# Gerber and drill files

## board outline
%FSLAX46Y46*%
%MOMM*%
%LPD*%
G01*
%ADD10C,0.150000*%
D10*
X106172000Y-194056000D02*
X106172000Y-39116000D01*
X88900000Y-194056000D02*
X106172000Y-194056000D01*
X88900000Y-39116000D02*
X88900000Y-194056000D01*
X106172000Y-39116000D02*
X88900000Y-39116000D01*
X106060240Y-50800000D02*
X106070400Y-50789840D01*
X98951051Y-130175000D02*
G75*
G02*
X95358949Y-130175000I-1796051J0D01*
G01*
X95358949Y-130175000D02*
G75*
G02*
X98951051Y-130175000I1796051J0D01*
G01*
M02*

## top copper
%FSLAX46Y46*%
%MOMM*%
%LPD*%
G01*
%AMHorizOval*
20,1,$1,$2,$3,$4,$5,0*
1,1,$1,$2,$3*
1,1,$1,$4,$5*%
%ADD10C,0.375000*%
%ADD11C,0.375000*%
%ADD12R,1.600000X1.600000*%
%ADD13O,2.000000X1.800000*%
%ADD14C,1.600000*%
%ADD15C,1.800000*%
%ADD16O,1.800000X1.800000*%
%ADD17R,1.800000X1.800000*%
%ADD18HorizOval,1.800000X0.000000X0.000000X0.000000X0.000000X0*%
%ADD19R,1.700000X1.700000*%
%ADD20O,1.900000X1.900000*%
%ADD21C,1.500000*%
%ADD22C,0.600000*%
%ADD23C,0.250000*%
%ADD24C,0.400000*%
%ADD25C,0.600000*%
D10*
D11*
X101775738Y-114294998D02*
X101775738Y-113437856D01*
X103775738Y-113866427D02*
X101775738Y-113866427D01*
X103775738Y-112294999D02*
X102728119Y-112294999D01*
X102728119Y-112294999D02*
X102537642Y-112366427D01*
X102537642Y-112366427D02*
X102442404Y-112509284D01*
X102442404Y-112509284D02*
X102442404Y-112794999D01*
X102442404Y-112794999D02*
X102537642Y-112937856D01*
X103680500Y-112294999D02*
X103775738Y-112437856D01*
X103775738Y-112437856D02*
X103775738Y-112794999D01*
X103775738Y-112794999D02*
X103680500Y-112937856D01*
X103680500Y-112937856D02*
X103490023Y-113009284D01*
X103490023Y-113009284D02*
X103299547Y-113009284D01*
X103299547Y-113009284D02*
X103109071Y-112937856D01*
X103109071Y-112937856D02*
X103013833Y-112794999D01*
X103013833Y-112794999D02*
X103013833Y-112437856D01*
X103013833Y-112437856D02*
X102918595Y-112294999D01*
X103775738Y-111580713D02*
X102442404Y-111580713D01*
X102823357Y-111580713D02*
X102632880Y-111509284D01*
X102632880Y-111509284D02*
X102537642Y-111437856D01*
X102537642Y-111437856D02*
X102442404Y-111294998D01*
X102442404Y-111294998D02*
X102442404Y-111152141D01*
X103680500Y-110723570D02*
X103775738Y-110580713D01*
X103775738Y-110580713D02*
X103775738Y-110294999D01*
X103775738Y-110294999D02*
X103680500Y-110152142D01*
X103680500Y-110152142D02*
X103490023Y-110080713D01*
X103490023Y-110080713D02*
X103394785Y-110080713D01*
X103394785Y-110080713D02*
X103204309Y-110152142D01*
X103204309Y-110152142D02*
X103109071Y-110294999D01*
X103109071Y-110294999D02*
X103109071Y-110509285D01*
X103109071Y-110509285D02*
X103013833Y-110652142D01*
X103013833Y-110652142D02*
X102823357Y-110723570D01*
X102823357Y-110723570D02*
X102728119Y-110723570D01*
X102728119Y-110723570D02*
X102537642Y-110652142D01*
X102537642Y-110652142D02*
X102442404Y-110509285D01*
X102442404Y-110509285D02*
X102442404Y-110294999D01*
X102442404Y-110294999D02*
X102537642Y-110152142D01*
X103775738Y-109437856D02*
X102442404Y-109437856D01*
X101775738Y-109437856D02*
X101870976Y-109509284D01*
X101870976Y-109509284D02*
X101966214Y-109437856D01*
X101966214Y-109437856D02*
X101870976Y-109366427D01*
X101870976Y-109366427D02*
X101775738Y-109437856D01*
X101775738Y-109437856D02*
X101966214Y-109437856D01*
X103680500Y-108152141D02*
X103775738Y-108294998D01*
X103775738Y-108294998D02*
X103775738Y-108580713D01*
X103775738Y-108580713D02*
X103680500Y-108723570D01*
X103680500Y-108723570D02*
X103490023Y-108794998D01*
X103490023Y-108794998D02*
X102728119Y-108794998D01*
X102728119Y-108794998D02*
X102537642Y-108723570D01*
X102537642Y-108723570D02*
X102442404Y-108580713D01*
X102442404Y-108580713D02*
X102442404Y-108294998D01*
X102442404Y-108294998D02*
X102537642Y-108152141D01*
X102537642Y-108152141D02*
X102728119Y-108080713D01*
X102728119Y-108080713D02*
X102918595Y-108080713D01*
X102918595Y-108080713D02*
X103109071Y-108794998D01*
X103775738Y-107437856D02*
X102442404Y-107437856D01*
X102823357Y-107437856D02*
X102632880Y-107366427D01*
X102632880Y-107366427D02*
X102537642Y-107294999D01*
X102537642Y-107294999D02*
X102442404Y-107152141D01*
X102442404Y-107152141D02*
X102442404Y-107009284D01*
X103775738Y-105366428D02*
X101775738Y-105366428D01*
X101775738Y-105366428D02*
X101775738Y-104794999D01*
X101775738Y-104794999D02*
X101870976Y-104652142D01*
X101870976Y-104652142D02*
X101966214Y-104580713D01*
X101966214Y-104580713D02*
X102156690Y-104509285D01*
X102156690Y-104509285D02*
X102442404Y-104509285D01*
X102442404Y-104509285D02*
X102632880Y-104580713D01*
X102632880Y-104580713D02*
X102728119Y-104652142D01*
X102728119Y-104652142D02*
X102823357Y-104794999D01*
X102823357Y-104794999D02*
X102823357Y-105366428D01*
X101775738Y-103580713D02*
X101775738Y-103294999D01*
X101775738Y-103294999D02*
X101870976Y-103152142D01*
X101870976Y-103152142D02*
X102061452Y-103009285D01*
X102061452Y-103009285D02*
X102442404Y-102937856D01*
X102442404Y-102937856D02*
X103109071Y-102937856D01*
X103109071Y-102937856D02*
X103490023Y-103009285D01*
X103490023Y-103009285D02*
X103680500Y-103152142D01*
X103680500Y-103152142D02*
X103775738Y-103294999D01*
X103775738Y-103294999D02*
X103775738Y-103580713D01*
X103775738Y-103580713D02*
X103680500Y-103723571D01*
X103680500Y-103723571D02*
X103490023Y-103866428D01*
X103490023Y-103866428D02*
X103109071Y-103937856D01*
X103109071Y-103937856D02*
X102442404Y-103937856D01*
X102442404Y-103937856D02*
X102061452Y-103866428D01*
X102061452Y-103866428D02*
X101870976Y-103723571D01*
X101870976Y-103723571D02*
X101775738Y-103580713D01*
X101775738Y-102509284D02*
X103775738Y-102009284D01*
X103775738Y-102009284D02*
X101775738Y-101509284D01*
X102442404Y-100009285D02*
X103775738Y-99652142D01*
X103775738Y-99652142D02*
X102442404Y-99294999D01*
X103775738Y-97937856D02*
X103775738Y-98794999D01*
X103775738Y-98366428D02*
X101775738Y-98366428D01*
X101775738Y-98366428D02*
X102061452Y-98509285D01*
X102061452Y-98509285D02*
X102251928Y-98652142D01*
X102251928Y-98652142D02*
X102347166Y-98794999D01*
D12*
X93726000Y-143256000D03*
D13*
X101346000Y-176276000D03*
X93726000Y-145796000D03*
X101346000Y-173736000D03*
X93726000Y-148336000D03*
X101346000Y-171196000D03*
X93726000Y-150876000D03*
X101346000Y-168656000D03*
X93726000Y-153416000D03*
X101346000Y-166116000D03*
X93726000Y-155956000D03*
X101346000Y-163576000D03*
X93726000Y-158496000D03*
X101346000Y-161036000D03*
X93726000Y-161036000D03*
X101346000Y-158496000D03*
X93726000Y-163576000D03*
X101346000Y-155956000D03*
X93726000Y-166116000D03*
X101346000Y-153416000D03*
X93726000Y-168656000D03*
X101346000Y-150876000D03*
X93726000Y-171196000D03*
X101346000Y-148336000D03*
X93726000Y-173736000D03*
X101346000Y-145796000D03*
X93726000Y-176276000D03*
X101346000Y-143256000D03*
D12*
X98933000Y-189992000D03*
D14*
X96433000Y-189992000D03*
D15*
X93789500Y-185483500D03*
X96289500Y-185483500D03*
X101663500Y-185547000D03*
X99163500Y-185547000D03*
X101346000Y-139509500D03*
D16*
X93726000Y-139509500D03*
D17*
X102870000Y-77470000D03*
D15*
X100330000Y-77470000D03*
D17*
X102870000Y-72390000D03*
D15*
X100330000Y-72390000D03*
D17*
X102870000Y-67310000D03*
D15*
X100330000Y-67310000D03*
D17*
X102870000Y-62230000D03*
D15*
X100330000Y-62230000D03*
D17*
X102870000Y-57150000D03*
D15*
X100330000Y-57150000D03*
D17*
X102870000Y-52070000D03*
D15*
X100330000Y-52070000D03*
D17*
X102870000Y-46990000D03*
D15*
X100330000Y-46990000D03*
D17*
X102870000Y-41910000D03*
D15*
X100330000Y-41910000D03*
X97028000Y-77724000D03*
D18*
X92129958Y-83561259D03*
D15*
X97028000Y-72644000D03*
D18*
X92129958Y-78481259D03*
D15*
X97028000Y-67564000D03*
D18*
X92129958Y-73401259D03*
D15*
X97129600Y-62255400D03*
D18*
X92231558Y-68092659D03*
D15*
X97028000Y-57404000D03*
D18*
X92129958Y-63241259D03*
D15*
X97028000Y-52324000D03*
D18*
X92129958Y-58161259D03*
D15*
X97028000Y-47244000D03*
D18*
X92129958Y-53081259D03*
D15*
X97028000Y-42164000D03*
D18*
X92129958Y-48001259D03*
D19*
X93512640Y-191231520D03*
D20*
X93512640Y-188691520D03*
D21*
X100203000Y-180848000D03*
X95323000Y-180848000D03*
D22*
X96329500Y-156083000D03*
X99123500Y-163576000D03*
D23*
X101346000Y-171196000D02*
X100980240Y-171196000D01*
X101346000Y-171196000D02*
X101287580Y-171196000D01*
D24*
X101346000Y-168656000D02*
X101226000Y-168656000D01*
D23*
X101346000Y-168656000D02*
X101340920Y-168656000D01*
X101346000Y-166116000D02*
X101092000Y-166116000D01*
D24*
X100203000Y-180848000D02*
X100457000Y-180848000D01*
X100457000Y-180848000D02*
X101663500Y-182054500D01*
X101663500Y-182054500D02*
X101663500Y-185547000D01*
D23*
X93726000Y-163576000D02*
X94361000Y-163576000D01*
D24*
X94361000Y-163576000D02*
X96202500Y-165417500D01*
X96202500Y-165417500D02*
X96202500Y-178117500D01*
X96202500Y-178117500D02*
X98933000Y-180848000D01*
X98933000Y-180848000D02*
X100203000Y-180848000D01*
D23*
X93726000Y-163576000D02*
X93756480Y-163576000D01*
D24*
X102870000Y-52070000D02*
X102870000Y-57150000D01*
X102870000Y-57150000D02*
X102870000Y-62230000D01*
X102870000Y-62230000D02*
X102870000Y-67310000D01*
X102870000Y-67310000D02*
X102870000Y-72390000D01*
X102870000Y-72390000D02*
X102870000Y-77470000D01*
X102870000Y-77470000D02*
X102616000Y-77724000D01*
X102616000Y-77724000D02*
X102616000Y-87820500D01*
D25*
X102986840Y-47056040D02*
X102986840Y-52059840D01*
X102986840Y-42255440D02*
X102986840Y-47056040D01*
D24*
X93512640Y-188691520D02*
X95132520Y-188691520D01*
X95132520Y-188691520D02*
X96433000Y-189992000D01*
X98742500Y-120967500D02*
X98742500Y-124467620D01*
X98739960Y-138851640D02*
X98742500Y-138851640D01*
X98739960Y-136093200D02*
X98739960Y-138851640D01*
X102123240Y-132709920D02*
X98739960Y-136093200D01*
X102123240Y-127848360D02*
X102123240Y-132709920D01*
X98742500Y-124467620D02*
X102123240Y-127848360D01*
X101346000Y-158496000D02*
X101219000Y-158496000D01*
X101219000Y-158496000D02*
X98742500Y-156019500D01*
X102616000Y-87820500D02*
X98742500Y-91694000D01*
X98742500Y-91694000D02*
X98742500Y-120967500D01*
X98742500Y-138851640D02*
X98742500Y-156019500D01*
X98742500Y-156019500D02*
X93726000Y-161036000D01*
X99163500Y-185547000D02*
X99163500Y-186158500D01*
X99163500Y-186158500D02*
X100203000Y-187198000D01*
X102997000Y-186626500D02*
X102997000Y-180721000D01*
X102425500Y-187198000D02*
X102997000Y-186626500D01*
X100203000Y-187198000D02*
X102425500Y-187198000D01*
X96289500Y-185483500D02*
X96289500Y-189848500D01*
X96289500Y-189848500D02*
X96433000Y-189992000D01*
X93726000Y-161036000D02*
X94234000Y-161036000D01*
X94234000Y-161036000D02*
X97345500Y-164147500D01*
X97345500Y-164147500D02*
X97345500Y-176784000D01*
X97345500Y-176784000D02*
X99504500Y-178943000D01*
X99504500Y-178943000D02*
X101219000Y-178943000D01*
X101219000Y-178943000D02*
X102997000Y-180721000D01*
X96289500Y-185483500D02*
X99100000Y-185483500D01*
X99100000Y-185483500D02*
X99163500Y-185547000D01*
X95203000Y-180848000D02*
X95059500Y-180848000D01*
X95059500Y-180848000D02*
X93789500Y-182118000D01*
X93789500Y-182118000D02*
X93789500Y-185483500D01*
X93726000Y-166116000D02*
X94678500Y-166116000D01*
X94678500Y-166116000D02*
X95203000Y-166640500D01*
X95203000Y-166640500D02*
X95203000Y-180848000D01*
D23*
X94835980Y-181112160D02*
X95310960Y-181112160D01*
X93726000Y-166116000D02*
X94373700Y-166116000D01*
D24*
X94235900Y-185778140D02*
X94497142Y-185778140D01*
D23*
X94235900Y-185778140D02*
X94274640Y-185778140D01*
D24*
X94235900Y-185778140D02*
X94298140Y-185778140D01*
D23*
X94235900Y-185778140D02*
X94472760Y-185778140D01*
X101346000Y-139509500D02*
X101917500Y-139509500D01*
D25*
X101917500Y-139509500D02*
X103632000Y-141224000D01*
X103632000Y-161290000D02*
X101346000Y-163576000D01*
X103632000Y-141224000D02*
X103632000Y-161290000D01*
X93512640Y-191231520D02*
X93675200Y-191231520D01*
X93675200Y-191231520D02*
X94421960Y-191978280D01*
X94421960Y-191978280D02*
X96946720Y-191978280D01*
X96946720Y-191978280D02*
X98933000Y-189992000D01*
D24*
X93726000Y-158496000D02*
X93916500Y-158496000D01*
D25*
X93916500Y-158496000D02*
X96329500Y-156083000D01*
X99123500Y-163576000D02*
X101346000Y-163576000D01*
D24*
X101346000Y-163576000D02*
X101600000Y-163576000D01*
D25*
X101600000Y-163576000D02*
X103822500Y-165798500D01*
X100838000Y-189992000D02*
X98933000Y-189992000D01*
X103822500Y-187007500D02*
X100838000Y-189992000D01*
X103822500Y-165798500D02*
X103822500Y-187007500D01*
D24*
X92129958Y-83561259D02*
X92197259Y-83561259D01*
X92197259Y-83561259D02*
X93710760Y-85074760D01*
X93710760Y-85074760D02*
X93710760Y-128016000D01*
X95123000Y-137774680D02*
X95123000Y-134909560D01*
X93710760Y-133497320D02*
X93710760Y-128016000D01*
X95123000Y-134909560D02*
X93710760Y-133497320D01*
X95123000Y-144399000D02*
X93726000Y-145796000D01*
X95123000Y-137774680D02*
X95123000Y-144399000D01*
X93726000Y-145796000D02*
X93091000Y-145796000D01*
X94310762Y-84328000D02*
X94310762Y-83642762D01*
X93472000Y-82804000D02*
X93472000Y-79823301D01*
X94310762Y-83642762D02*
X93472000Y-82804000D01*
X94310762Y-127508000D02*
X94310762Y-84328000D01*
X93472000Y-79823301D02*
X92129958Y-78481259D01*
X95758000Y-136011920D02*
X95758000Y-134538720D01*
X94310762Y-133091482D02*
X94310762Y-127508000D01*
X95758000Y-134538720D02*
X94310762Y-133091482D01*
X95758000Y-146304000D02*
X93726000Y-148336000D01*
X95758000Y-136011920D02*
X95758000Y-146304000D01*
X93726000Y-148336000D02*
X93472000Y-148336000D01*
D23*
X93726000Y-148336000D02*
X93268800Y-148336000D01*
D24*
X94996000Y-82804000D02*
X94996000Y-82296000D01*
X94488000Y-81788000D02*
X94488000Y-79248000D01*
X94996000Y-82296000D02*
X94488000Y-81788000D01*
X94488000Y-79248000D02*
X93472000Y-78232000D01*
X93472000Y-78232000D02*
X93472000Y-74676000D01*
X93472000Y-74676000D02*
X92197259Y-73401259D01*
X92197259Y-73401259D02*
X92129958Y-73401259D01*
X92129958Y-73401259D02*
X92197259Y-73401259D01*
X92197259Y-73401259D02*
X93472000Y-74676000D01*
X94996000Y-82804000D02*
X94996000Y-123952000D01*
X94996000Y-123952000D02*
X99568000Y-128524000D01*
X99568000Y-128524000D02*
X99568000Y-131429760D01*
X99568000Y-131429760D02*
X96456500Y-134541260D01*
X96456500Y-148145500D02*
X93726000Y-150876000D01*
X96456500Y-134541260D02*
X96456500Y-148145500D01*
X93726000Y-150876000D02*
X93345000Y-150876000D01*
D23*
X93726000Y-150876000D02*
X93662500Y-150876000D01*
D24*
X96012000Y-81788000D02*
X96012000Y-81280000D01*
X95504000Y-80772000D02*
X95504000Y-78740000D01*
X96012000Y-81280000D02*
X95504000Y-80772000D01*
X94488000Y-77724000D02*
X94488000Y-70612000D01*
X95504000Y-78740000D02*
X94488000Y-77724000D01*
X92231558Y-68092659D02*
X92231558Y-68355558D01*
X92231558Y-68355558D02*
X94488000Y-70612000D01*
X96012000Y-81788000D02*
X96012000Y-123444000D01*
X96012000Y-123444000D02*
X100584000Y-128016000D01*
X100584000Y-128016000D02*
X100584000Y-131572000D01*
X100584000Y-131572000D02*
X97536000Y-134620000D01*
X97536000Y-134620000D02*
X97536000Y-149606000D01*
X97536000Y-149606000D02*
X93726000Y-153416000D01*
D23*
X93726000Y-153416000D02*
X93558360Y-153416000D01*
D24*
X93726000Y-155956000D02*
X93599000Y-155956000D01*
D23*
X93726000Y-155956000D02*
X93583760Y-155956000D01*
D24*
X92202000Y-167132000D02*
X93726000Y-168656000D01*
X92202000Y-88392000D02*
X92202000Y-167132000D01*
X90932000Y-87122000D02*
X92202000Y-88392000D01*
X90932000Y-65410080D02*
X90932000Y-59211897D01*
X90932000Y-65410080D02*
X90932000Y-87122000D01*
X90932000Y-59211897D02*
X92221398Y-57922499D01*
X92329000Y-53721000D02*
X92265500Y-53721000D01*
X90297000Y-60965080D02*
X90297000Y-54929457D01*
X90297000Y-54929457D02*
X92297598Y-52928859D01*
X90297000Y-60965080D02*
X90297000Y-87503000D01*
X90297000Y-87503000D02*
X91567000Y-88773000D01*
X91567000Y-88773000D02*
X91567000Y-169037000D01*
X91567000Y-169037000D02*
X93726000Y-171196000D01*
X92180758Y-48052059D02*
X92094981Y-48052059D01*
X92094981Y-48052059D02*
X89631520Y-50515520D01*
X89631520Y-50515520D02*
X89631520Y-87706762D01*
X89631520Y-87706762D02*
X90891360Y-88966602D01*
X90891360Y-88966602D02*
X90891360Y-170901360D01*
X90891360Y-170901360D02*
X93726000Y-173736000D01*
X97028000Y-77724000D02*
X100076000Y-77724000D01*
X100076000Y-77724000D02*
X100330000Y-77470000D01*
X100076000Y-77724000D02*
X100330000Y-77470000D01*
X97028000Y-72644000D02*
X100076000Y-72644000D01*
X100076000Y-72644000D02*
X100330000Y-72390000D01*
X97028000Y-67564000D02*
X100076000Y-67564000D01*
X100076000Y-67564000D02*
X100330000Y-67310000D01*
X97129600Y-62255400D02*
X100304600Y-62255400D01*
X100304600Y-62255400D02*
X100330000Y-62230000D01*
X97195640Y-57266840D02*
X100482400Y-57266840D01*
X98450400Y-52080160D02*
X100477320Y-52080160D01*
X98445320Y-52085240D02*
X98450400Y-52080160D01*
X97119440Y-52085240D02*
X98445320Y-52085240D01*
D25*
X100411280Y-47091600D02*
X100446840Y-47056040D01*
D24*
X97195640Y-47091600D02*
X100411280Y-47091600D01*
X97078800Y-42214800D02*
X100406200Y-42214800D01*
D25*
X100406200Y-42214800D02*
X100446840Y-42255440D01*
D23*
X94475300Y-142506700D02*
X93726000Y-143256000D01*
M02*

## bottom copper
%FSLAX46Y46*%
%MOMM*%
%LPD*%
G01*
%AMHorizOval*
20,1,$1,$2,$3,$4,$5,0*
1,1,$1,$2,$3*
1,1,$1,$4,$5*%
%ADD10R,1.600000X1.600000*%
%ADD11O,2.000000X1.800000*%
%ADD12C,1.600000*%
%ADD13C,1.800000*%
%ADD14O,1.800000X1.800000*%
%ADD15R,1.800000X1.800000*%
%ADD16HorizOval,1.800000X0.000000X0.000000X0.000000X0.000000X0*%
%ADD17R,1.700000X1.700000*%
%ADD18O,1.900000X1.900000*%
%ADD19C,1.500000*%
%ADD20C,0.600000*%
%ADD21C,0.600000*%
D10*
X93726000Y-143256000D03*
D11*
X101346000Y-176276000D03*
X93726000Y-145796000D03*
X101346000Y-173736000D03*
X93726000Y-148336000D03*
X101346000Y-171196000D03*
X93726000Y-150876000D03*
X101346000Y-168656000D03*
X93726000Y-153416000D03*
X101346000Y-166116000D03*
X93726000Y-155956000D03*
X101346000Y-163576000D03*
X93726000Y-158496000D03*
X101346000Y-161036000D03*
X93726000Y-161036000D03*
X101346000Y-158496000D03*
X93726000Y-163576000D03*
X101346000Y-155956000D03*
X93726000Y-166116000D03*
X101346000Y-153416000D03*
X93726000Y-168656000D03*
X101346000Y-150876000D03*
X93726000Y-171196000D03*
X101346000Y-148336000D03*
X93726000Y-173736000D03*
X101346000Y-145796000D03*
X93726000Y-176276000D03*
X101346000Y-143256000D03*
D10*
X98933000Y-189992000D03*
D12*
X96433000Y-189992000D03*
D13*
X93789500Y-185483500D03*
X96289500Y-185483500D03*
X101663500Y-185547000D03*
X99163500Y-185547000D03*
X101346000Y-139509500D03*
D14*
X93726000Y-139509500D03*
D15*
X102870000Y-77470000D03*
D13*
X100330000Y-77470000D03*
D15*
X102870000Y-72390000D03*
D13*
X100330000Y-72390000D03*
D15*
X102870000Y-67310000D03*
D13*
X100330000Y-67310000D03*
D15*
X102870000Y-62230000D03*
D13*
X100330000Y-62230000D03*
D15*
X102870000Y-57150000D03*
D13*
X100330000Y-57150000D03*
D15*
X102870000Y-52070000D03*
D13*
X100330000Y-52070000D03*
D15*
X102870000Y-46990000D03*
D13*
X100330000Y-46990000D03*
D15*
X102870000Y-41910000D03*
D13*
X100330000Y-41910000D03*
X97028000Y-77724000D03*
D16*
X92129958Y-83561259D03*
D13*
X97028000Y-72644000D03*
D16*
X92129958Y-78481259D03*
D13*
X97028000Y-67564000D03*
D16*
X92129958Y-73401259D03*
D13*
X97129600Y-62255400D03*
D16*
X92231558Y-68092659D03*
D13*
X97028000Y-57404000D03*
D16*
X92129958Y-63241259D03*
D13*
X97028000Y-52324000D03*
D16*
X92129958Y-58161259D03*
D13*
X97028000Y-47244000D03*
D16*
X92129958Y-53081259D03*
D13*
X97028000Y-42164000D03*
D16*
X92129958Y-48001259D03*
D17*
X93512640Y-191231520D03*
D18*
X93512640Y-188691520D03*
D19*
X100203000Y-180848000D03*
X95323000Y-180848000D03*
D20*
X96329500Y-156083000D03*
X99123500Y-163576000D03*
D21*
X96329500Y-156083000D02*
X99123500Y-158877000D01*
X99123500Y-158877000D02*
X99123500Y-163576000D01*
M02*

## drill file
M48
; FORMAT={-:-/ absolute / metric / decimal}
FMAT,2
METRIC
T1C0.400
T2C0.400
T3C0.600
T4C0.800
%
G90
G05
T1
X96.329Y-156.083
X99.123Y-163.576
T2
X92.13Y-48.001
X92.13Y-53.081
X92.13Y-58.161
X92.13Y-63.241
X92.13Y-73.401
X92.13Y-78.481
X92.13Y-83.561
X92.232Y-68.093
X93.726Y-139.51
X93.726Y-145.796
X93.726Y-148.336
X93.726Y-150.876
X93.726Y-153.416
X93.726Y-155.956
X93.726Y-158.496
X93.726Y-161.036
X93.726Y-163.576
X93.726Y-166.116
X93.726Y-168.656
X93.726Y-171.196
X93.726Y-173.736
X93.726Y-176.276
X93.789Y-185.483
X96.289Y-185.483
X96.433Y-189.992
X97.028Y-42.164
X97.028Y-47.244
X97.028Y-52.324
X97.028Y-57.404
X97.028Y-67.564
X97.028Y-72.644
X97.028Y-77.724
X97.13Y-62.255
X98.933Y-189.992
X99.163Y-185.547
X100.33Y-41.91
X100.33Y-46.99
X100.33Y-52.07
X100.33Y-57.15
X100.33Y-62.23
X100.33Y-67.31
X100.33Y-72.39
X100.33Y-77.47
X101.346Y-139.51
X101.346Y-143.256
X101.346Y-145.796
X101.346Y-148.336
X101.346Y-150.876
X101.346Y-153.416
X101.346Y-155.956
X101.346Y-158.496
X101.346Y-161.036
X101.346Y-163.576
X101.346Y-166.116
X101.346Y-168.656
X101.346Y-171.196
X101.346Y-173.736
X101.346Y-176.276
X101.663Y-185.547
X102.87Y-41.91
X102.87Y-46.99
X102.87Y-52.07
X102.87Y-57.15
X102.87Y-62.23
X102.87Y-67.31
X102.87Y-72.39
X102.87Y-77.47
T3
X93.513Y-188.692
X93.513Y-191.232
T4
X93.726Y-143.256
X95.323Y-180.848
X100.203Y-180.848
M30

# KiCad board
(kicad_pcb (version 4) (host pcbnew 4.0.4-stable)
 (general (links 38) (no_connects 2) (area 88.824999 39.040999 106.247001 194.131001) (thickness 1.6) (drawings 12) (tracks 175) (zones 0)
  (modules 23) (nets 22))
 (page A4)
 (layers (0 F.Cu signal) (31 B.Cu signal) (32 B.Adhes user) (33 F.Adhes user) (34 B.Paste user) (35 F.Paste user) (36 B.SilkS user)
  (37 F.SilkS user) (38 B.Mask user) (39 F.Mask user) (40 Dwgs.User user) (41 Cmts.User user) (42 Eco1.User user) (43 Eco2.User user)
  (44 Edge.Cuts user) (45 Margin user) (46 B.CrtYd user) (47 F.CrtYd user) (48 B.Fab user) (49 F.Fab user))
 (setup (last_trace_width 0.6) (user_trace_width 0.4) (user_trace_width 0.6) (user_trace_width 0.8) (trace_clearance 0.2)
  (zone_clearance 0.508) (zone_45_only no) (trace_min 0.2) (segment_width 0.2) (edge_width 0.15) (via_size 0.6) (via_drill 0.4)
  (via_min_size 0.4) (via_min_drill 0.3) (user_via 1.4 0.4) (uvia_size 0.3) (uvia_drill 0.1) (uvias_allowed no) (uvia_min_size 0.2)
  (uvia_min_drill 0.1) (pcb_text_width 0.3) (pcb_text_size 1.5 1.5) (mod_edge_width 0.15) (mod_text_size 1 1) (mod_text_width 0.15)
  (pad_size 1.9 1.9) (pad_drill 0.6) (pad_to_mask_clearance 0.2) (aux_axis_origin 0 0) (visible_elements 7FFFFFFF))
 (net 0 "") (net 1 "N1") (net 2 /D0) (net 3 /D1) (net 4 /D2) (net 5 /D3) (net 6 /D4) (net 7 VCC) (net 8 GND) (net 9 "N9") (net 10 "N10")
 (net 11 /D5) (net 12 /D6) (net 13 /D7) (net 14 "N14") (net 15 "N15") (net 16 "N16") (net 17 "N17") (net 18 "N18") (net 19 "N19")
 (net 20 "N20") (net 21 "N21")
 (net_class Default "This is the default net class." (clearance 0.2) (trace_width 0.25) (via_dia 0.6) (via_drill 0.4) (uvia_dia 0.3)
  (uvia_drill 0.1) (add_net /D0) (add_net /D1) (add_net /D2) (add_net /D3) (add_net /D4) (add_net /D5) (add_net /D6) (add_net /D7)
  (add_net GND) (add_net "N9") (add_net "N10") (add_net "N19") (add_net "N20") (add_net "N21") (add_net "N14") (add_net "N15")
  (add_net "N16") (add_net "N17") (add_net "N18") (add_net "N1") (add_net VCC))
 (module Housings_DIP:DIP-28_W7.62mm (layer F.Cu) (at 93.726 143.256)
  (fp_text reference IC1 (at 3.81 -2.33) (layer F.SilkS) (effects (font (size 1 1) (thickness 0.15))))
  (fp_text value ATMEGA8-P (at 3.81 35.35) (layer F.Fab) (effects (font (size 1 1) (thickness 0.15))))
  (pad 1 thru_hole rect (at 0 0) (size 1.6 1.6) (drill 0.8) (layers *.Cu *.Mask) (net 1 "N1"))
  (pad 15 thru_hole oval (at 7.62 33.02) (size 2 1.8) (drill 0.4) (layers *.Cu *.Mask))
  (pad 2 thru_hole oval (at 0 2.54) (size 2 1.8) (drill 0.4) (layers *.Cu *.Mask) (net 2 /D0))
  (pad 16 thru_hole oval (at 7.62 30.48) (size 2 1.8) (drill 0.4) (layers *.Cu *.Mask))
  (pad 3 thru_hole oval (at 0 5.08) (size 2 1.8) (drill 0.4) (layers *.Cu *.Mask) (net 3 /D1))
  (pad 17 thru_hole oval (at 7.62 27.94) (size 2 1.8) (drill 0.4) (layers *.Cu *.Mask))
  (pad 4 thru_hole oval (at 0 7.62) (size 2 1.8) (drill 0.4) (layers *.Cu *.Mask) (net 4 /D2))
  (pad 18 thru_hole oval (at 7.62 25.4) (size 2 1.8) (drill 0.4) (layers *.Cu *.Mask))
  (pad 5 thru_hole oval (at 0 10.16) (size 2 1.8) (drill 0.4) (layers *.Cu *.Mask) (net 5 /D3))
  (pad 19 thru_hole oval (at 7.62 22.86) (size 2 1.8) (drill 0.4) (layers *.Cu *.Mask))
  (pad 6 thru_hole oval (at 0 12.7) (size 2 1.8) (drill 0.4) (layers *.Cu *.Mask) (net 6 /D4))
  (pad 20 thru_hole oval (at 7.62 20.32) (size 2 1.8) (drill 0.4) (layers *.Cu *.Mask) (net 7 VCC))
  (pad 7 thru_hole oval (at 0 15.24) (size 2 1.8) (drill 0.4) (layers *.Cu *.Mask) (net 7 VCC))
  (pad 21 thru_hole oval (at 7.62 17.78) (size 2 1.8) (drill 0.4) (layers *.Cu *.Mask))
  (pad 8 thru_hole oval (at 0 17.78) (size 2 1.8) (drill 0.4) (layers *.Cu *.Mask) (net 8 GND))
  (pad 22 thru_hole oval (at 7.62 15.24) (size 2 1.8) (drill 0.4) (layers *.Cu *.Mask) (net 8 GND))
  (pad 9 thru_hole oval (at 0 20.32) (size 2 1.8) (drill 0.4) (layers *.Cu *.Mask) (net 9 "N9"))
  (pad 23 thru_hole oval (at 7.62 12.7) (size 2 1.8) (drill 0.4) (layers *.Cu *.Mask))
  (pad 10 thru_hole oval (at 0 22.86) (size 2 1.8) (drill 0.4) (layers *.Cu *.Mask) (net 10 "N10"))
  (pad 24 thru_hole oval (at 7.62 10.16) (size 2 1.8) (drill 0.4) (layers *.Cu *.Mask))
  (pad 11 thru_hole oval (at 0 25.4) (size 2 1.8) (drill 0.4) (layers *.Cu *.Mask) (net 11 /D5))
  (pad 25 thru_hole oval (at 7.62 7.62) (size 2 1.8) (drill 0.4) (layers *.Cu *.Mask))
  (pad 12 thru_hole oval (at 0 27.94) (size 2 1.8) (drill 0.4) (layers *.Cu *.Mask) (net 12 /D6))
  (pad 26 thru_hole oval (at 7.62 5.08) (size 2 1.8) (drill 0.4) (layers *.Cu *.Mask))
  (pad 13 thru_hole oval (at 0 30.48) (size 2 1.8) (drill 0.4) (layers *.Cu *.Mask) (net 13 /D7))
  (pad 27 thru_hole oval (at 7.62 2.54) (size 2 1.8) (drill 0.4) (layers *.Cu *.Mask))
  (pad 14 thru_hole oval (at 0 33.02) (size 2 1.8) (drill 0.4) (layers *.Cu *.Mask))
  (pad 28 thru_hole oval (at 7.62 0) (size 2 1.8) (drill 0.4) (layers *.Cu *.Mask)))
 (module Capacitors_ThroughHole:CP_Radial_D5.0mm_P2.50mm (layer F.Cu) (at 98.933 189.992 180)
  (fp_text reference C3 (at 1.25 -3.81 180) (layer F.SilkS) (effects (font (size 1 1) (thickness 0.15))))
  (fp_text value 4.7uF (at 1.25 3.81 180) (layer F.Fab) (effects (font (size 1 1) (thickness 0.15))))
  (pad 1 thru_hole rect (at 0 0 180) (size 1.6 1.6) (drill 0.4) (layers *.Cu *.Mask) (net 7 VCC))
  (pad 2 thru_hole circle (at 2.5 0 180) (size 1.6 1.6) (drill 0.4) (layers *.Cu *.Mask) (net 8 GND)))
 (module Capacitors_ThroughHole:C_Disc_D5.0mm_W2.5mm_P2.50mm (layer F.Cu) (at 93.7895 185.4835)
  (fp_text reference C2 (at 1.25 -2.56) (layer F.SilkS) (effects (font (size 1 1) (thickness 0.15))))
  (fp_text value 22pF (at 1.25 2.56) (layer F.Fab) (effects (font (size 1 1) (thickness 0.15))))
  (pad 1 thru_hole circle (at 0 0) (size 1.8 1.8) (drill 0.4) (layers *.Cu *.Mask) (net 10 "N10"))
  (pad 2 thru_hole circle (at 2.5 0) (size 1.8 1.8) (drill 0.4) (layers *.Cu *.Mask) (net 8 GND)))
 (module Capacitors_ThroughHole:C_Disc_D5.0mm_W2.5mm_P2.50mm (layer F.Cu) (at 101.6635 185.547 180)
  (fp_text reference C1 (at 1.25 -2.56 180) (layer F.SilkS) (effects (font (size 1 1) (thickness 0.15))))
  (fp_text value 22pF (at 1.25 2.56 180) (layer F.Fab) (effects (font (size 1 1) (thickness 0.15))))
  (pad 1 thru_hole circle (at 0 0 180) (size 1.8 1.8) (drill 0.4) (layers *.Cu *.Mask) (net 9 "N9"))
  (pad 2 thru_hole circle (at 2.5 0 180) (size 1.8 1.8) (drill 0.4) (layers *.Cu *.Mask) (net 8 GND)))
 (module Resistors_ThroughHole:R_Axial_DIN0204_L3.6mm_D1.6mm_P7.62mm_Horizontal (layer F.Cu) (at 101.346 139.5095 180)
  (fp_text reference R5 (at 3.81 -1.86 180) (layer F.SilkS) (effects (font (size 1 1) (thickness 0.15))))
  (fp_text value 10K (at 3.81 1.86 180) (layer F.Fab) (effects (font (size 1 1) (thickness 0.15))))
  (pad 1 thru_hole circle (at 0 0 180) (size 1.8 1.8) (drill 0.4) (layers *.Cu *.Mask) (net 7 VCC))
  (pad 2 thru_hole oval (at 7.62 0 180) (size 1.8 1.8) (drill 0.4) (layers *.Cu *.Mask) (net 1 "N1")))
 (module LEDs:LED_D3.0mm (layer F.Cu) (at 102.87 77.47 180)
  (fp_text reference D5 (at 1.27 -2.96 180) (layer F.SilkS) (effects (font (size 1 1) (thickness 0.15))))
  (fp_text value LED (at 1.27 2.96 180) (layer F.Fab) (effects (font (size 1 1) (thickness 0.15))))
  (pad 1 thru_hole rect (at 0 0 180) (size 1.8 1.8) (drill 0.4) (layers *.Cu *.Mask) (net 8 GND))
  (pad 2 thru_hole circle (at 2.54 0 180) (size 1.8 1.8) (drill 0.4) (layers *.Cu *.Mask) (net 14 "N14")))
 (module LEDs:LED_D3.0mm (layer F.Cu) (at 102.87 72.39 180)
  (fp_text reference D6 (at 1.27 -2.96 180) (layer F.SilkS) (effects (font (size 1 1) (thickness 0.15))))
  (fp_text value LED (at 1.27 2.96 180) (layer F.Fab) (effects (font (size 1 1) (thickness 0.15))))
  (pad 1 thru_hole rect (at 0 0 180) (size 1.8 1.8) (drill 0.4) (layers *.Cu *.Mask) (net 8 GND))
  (pad 2 thru_hole circle (at 2.54 0 180) (size 1.8 1.8) (drill 0.4) (layers *.Cu *.Mask) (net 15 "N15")))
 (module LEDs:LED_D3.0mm (layer F.Cu) (at 102.87 67.31 180)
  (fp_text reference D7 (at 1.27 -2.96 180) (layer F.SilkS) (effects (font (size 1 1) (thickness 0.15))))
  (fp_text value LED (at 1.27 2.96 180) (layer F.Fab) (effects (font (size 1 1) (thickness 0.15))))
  (pad 1 thru_hole rect (at 0 0 180) (size 1.8 1.8) (drill 0.4) (layers *.Cu *.Mask) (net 8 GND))
  (pad 2 thru_hole circle (at 2.54 0 180) (size 1.8 1.8) (drill 0.4) (layers *.Cu *.Mask) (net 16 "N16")))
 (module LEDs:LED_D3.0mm (layer F.Cu) (at 102.87 62.23 180)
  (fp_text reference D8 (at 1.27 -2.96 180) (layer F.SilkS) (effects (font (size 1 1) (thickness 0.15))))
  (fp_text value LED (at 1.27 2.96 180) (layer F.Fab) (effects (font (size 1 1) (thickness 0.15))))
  (pad 1 thru_hole rect (at 0 0 180) (size 1.8 1.8) (drill 0.4) (layers *.Cu *.Mask) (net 8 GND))
  (pad 2 thru_hole circle (at 2.54 0 180) (size 1.8 1.8) (drill 0.4) (layers *.Cu *.Mask) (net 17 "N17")))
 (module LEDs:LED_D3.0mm (layer F.Cu) (at 102.87 57.15 180)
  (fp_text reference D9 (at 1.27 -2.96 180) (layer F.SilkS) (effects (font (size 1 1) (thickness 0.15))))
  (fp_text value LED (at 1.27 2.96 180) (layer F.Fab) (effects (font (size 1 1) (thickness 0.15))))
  (pad 1 thru_hole rect (at 0 0 180) (size 1.8 1.8) (drill 0.4) (layers *.Cu *.Mask) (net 8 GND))
  (pad 2 thru_hole circle (at 2.54 0 180) (size 1.8 1.8) (drill 0.4) (layers *.Cu *.Mask) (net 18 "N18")))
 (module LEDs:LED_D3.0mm (layer F.Cu) (at 102.87 52.07 180)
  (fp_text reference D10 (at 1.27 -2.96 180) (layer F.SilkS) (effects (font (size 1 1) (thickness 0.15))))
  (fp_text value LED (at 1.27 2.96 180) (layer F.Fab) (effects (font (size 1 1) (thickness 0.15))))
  (pad 1 thru_hole rect (at 0 0 180) (size 1.8 1.8) (drill 0.4) (layers *.Cu *.Mask) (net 8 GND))
  (pad 2 thru_hole circle (at 2.54 0 180) (size 1.8 1.8) (drill 0.4) (layers *.Cu *.Mask) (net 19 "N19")))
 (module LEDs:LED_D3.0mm (layer F.Cu) (at 102.87 46.99 180)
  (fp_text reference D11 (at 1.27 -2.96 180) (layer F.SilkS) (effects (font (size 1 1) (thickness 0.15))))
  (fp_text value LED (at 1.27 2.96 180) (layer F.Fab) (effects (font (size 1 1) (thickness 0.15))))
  (pad 1 thru_hole rect (at 0 0 180) (size 1.8 1.8) (drill 0.4) (layers *.Cu *.Mask) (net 8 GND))
  (pad 2 thru_hole circle (at 2.54 0 180) (size 1.8 1.8) (drill 0.4) (layers *.Cu *.Mask) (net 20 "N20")))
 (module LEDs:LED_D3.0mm (layer F.Cu) (at 102.87 41.91 180)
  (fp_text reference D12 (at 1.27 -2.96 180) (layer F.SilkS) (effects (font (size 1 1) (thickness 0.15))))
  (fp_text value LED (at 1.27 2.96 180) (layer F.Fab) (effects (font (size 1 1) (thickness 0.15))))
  (pad 1 thru_hole rect (at 0 0 180) (size 1.8 1.8) (drill 0.4) (layers *.Cu *.Mask) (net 8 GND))
  (pad 2 thru_hole circle (at 2.54 0 180) (size 1.8 1.8) (drill 0.4) (layers *.Cu *.Mask) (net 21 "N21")))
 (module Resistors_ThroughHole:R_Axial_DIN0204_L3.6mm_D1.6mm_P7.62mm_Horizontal (layer F.Cu) (at 97.028 77.724 230)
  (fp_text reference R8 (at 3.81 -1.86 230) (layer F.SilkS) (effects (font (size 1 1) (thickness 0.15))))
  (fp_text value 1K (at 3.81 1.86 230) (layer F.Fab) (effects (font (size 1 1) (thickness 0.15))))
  (pad 1 thru_hole circle (at 0 0 230) (size 1.8 1.8) (drill 0.4) (layers *.Cu *.Mask) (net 14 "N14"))
  (pad 2 thru_hole oval (at 7.62 0 230) (size 1.8 1.8) (drill 0.4) (layers *.Cu *.Mask) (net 2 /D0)))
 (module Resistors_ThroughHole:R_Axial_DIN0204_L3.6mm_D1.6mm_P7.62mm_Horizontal (layer F.Cu) (at 97.028 72.644 230)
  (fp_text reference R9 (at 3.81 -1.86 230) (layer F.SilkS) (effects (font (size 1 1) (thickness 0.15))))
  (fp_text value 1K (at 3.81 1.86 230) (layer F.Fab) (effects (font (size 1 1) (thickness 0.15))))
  (pad 1 thru_hole circle (at 0 0 230) (size 1.8 1.8) (drill 0.4) (layers *.Cu *.Mask) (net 15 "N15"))
  (pad 2 thru_hole oval (at 7.62 0 230) (size 1.8 1.8) (drill 0.4) (layers *.Cu *.Mask) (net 3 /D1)))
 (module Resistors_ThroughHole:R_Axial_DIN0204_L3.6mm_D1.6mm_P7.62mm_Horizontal (layer F.Cu) (at 97.028 67.564 230)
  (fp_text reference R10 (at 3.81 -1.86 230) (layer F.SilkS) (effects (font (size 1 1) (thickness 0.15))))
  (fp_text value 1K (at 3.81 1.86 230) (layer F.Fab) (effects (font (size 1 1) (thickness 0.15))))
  (pad 1 thru_hole circle (at 0 0 230) (size 1.8 1.8) (drill 0.4) (layers *.Cu *.Mask) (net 16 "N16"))
  (pad 2 thru_hole oval (at 7.62 0 230) (size 1.8 1.8) (drill 0.4) (layers *.Cu *.Mask) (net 4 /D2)))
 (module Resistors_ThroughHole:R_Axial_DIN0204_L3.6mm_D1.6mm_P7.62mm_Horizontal (layer F.Cu) (at 97.1296 62.2554 230)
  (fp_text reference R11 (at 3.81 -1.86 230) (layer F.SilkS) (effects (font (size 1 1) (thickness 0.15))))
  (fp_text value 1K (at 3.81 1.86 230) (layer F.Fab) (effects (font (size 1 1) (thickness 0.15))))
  (pad 1 thru_hole circle (at 0 0 230) (size 1.8 1.8) (drill 0.4) (layers *.Cu *.Mask) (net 17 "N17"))
  (pad 2 thru_hole oval (at 7.62 0 230) (size 1.8 1.8) (drill 0.4) (layers *.Cu *.Mask) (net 5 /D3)))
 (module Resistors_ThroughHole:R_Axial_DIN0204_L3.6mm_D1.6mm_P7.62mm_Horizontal (layer F.Cu) (at 97.028 57.404 230)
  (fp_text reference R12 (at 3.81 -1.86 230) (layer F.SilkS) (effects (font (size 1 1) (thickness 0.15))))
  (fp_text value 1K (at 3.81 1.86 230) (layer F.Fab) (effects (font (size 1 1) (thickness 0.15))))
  (pad 1 thru_hole circle (at 0 0 230) (size 1.8 1.8) (drill 0.4) (layers *.Cu *.Mask) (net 18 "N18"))
  (pad 2 thru_hole oval (at 7.62 0 230) (size 1.8 1.8) (drill 0.4) (layers *.Cu *.Mask) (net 6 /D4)))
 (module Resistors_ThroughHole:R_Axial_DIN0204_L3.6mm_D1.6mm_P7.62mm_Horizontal (layer F.Cu) (at 97.028 52.324 230)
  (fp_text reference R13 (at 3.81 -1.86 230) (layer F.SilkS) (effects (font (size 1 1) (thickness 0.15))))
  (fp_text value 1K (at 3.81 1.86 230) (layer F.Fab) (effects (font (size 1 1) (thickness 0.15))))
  (pad 1 thru_hole circle (at 0 0 230) (size 1.8 1.8) (drill 0.4) (layers *.Cu *.Mask) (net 19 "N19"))
  (pad 2 thru_hole oval (at 7.62 0 230) (size 1.8 1.8) (drill 0.4) (layers *.Cu *.Mask) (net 11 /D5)))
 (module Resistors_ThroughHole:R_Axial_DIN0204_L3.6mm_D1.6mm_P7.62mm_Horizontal (layer F.Cu) (at 97.028 47.244 230)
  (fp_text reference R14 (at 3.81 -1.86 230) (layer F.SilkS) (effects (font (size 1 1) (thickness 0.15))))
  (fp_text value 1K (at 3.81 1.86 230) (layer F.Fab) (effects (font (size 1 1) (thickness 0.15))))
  (pad 1 thru_hole circle (at 0 0 230) (size 1.8 1.8) (drill 0.4) (layers *.Cu *.Mask) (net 20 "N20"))
  (pad 2 thru_hole oval (at 7.62 0 230) (size 1.8 1.8) (drill 0.4) (layers *.Cu *.Mask) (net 12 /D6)))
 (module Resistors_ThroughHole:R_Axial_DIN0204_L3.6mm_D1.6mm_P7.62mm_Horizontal (layer F.Cu) (at 97.028 42.164 230)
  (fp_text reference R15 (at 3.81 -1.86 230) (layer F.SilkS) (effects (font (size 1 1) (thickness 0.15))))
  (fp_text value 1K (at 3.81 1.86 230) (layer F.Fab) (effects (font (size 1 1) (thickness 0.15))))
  (pad 1 thru_hole circle (at 0 0 230) (size 1.8 1.8) (drill 0.4) (layers *.Cu *.Mask) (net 21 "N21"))
  (pad 2 thru_hole oval (at 7.62 0 230) (size 1.8 1.8) (drill 0.4) (layers *.Cu *.Mask) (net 13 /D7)))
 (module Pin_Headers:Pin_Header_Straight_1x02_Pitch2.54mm (layer F.Cu) (at 93.51264 191.23152 180)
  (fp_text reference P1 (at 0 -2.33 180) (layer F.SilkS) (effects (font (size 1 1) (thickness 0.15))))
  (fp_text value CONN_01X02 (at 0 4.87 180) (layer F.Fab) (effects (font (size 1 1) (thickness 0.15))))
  (pad 1 thru_hole rect (at 0 0 180) (size 1.7 1.7) (drill 0.6) (layers *.Cu *.Mask) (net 7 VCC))
  (pad 2 thru_hole oval (at 0 2.54 180) (size 1.9 1.9) (drill 0.6) (layers *.Cu *.Mask) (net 8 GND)))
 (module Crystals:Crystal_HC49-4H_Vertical (layer F.Cu) (at 100.203 180.848 180)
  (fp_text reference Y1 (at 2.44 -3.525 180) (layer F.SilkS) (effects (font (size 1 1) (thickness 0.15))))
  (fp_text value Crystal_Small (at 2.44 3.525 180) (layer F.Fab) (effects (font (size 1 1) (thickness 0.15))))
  (pad 1 thru_hole circle (at 0 0 180) (size 1.5 1.5) (drill 0.8) (layers *.Cu *.Mask) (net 9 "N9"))
  (pad 2 thru_hole circle (at 4.88 0 180) (size 1.5 1.5) (drill 0.8) (layers *.Cu *.Mask) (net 10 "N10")))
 (gr_line (start 106.172 194.056) (end 106.172 39.116) (angle 90) (layer Edge.Cuts) (width 0.15))
 (gr_line (start 88.9 194.056) (end 106.172 194.056) (angle 90) (layer Edge.Cuts) (width 0.15))
 (gr_line (start 88.9 39.116) (end 88.9 194.056) (angle 90) (layer Edge.Cuts) (width 0.15))
 (gr_line (start 106.172 39.116) (end 88.9 39.116) (angle 90) (layer Edge.Cuts) (width 0.15))
 (gr_line (start 106.06024 50.8) (end 106.0704 50.78984) (angle 90) (layer Edge.Cuts) (width 0.15))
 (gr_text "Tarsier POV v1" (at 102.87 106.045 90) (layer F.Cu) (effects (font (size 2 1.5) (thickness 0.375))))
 (gr_circle (center 97.155 130.175) (end 98.425 131.445) (layer Edge.Cuts) (width 0.15))
 (segment (start 101.346 171.196) (end 100.98024 171.196) (width 0.25) (layer F.Cu) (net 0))
 (segment (start 101.346 171.196) (end 101.28758 171.196) (width 0.25) (layer F.Cu) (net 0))
 (segment (start 101.346 168.656) (end 101.226 168.656) (width 0.4) (layer F.Cu) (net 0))
 (segment (start 101.346 168.656) (end 101.34092 168.656) (width 0.25) (layer F.Cu) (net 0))
 (segment (start 101.346 166.116) (end 101.092 166.116) (width 0.25) (layer F.Cu) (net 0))
 (segment (start 100.203 180.848) (end 100.457 180.848) (width 0.4) (layer F.Cu) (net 9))
 (segment (start 100.457 180.848) (end 101.6635 182.0545) (width 0.4) (layer F.Cu) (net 9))
 (segment (start 101.6635 182.0545) (end 101.6635 185.547) (width 0.4) (layer F.Cu) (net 9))
 (segment (start 93.726 163.576) (end 94.361 163.576) (width 0.25) (layer F.Cu) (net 9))
 (segment (start 94.361 163.576) (end 96.2025 165.4175) (width 0.4) (layer F.Cu) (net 9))
 (segment (start 96.2025 165.4175) (end 96.2025 178.1175) (width 0.4) (layer F.Cu) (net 9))
 (segment (start 96.2025 178.1175) (end 98.933 180.848) (width 0.4) (layer F.Cu) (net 9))
 (segment (start 98.933 180.848) (end 100.203 180.848) (width 0.4) (layer F.Cu) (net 9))
 (segment (start 93.726 163.576) (end 93.75648 163.576) (width 0.25) (layer F.Cu) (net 9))
 (segment (start 102.87 52.07) (end 102.87 57.15) (width 0.4) (layer F.Cu) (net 8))
 (segment (start 102.87 57.15) (end 102.87 62.23) (width 0.4) (layer F.Cu) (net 8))
 (segment (start 102.87 62.23) (end 102.87 67.31) (width 0.4) (layer F.Cu) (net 8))
 (segment (start 102.87 67.31) (end 102.87 72.39) (width 0.4) (layer F.Cu) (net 8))
 (segment (start 102.87 72.39) (end 102.87 77.47) (width 0.4) (layer F.Cu) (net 8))
 (segment (start 102.87 77.47) (end 102.616 77.724) (width 0.4) (layer F.Cu) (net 8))
 (segment (start 102.616 77.724) (end 102.616 87.8205) (width 0.4) (layer F.Cu) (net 8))
 (segment (start 102.98684 47.05604) (end 102.98684 52.05984) (width 0.6) (layer F.Cu) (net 8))
 (segment (start 102.98684 42.25544) (end 102.98684 47.05604) (width 0.6) (layer F.Cu) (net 8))
 (segment (start 93.51264 188.69152) (end 95.13252 188.69152) (width 0.4) (layer F.Cu) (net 8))
 (segment (start 95.13252 188.69152) (end 96.433 189.992) (width 0.4) (layer F.Cu) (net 8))
 (segment (start 98.7425 120.9675) (end 98.7425 124.46762) (width 0.4) (layer F.Cu) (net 8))
 (segment (start 98.73996 138.85164) (end 98.7425 138.85164) (width 0.4) (layer F.Cu) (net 8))
 (segment (start 98.73996 136.0932) (end 98.73996 138.85164) (width 0.4) (layer F.Cu) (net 8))
 (segment (start 102.12324 132.70992) (end 98.73996 136.0932) (width 0.4) (layer F.Cu) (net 8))
 (segment (start 102.12324 127.84836) (end 102.12324 132.70992) (width 0.4) (layer F.Cu) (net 8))
 (segment (start 98.7425 124.46762) (end 102.12324 127.84836) (width 0.4) (layer F.Cu) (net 8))
 (segment (start 101.346 158.496) (end 101.219 158.496) (width 0.4) (layer F.Cu) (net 8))
 (segment (start 101.219 158.496) (end 98.7425 156.0195) (width 0.4) (layer F.Cu) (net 8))
 (segment (start 102.616 87.8205) (end 98.7425 91.694) (width 0.4) (layer F.Cu) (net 8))
 (segment (start 98.7425 91.694) (end 98.7425 120.9675) (width 0.4) (layer F.Cu) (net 8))
 (segment (start 98.7425 138.85164) (end 98.7425 156.0195) (width 0.4) (layer F.Cu) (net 8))
 (segment (start 98.7425 156.0195) (end 93.726 161.036) (width 0.4) (layer F.Cu) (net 8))
 (segment (start 99.1635 185.547) (end 99.1635 186.1585) (width 0.4) (layer F.Cu) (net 8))
 (segment (start 99.1635 186.1585) (end 100.203 187.198) (width 0.4) (layer F.Cu) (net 8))
 (segment (start 102.997 186.6265) (end 102.997 180.721) (width 0.4) (layer F.Cu) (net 8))
 (segment (start 102.4255 187.198) (end 102.997 186.6265) (width 0.4) (layer F.Cu) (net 8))
 (segment (start 100.203 187.198) (end 102.4255 187.198) (width 0.4) (layer F.Cu) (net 8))
 (segment (start 96.2895 185.4835) (end 96.2895 189.8485) (width 0.4) (layer F.Cu) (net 8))
 (segment (start 96.2895 189.8485) (end 96.433 189.992) (width 0.4) (layer F.Cu) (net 8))
 (segment (start 93.726 161.036) (end 94.234 161.036) (width 0.4) (layer F.Cu) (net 8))
 (segment (start 94.234 161.036) (end 97.3455 164.1475) (width 0.4) (layer F.Cu) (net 8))
 (segment (start 97.3455 164.1475) (end 97.3455 176.784) (width 0.4) (layer F.Cu) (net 8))
 (segment (start 97.3455 176.784) (end 99.5045 178.943) (width 0.4) (layer F.Cu) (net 8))
 (segment (start 99.5045 178.943) (end 101.219 178.943) (width 0.4) (layer F.Cu) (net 8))
 (segment (start 101.219 178.943) (end 102.997 180.721) (width 0.4) (layer F.Cu) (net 8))
 (segment (start 96.2895 185.4835) (end 99.1 185.4835) (width 0.4) (layer F.Cu) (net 8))
 (segment (start 99.1 185.4835) (end 99.1635 185.547) (width 0.4) (layer F.Cu) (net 8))
 (segment (start 95.203 180.848) (end 95.0595 180.848) (width 0.4) (layer F.Cu) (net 10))
 (segment (start 95.0595 180.848) (end 93.7895 182.118) (width 0.4) (layer F.Cu) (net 10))
 (segment (start 93.7895 182.118) (end 93.7895 185.4835) (width 0.4) (layer F.Cu) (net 10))
 (segment (start 93.726 166.116) (end 94.6785 166.116) (width 0.4) (layer F.Cu) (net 10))
 (segment (start 94.6785 166.116) (end 95.203 166.6405) (width 0.4) (layer F.Cu) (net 10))
 (segment (start 95.203 166.6405) (end 95.203 180.848) (width 0.4) (layer F.Cu) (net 10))
 (segment (start 94.83598 181.11216) (end 95.31096 181.11216) (width 0.25) (layer F.Cu) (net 10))
 (segment (start 93.726 166.116) (end 94.3737 166.116) (width 0.25) (layer F.Cu) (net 10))
 (segment (start 94.2359 185.77814) (end 94.497142 185.77814) (width 0.4) (layer F.Cu) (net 10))
 (segment (start 94.2359 185.77814) (end 94.27464 185.77814) (width 0.25) (layer F.Cu) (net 10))
 (segment (start 94.2359 185.77814) (end 94.29814 185.77814) (width 0.4) (layer F.Cu) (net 10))
 (segment (start 94.2359 185.77814) (end 94.47276 185.77814) (width 0.25) (layer F.Cu) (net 10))
 (segment (start 101.346 139.5095) (end 101.9175 139.5095) (width 0.25) (layer F.Cu) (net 7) (status C00000))
 (segment (start 101.9175 139.5095) (end 103.632 141.224) (width 0.6) (layer F.Cu) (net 7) (status 400000))
 (segment (start 103.632 161.29) (end 101.346 163.576) (width 0.6) (layer F.Cu) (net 7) (status 800000))
 (segment (start 103.632 141.224) (end 103.632 161.29) (width 0.6) (layer F.Cu) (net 7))
 (segment (start 93.51264 191.23152) (end 93.6752 191.23152) (width 0.6) (layer F.Cu) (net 7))
 (segment (start 93.6752 191.23152) (end 94.42196 191.97828) (width 0.6) (layer F.Cu) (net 7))
 (segment (start 94.42196 191.97828) (end 96.94672 191.97828) (width 0.6) (layer F.Cu) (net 7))
 (segment (start 96.94672 191.97828) (end 98.933 189.992) (width 0.6) (layer F.Cu) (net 7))
 (segment (start 93.726 158.496) (end 93.9165 158.496) (width 0.4) (layer F.Cu) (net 7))
 (segment (start 93.9165 158.496) (end 96.3295 156.083) (width 0.6) (layer F.Cu) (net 7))
 (via (at 96.3295 156.083) (size 0.6) (drill 0.4) (layers F.Cu B.Cu) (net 7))
 (segment (start 96.3295 156.083) (end 99.1235 158.877) (width 0.6) (layer B.Cu) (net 7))
 (segment (start 99.1235 158.877) (end 99.1235 163.576) (width 0.6) (layer B.Cu) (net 7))
 (via (at 99.1235 163.576) (size 0.6) (drill 0.4) (layers F.Cu B.Cu) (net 7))
 (segment (start 99.1235 163.576) (end 101.346 163.576) (width 0.6) (layer F.Cu) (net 7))
 (segment (start 101.346 163.576) (end 101.6 163.576) (width 0.4) (layer F.Cu) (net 7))
 (segment (start 101.6 163.576) (end 103.8225 165.7985) (width 0.6) (layer F.Cu) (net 7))
 (segment (start 100.838 189.992) (end 98.933 189.992) (width 0.6) (layer F.Cu) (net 7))
 (segment (start 103.8225 187.0075) (end 100.838 189.992) (width 0.6) (layer F.Cu) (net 7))
 (segment (start 103.8225 165.7985) (end 103.8225 187.0075) (width 0.6) (layer F.Cu) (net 7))
 (segment (start 92.129958 83.561259) (end 92.197259 83.561259) (width 0.4) (layer F.Cu) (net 2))
 (segment (start 92.197259 83.561259) (end 93.71076 85.07476) (width 0.4) (layer F.Cu) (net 2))
 (segment (start 93.71076 85.07476) (end 93.71076 128.016) (width 0.4) (layer F.Cu) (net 2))
 (segment (start 95.123 137.77468) (end 95.123 134.90956) (width 0.4) (layer F.Cu) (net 2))
 (segment (start 93.71076 133.49732) (end 93.71076 128.016) (width 0.4) (layer F.Cu) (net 2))
 (segment (start 95.123 134.90956) (end 93.71076 133.49732) (width 0.4) (layer F.Cu) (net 2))
 (segment (start 95.123 144.399) (end 93.726 145.796) (width 0.4) (layer F.Cu) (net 2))
 (segment (start 95.123 137.77468) (end 95.123 144.399) (width 0.4) (layer F.Cu) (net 2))
 (segment (start 93.726 145.796) (end 93.091 145.796) (width 0.4) (layer F.Cu) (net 2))
 (segment (start 94.310762 84.328) (end 94.310762 83.642762) (width 0.4) (layer F.Cu) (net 3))
 (segment (start 93.472 82.804) (end 93.472 79.823301) (width 0.4) (layer F.Cu) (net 3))
 (segment (start 94.310762 83.642762) (end 93.472 82.804) (width 0.4) (layer F.Cu) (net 3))
 (segment (start 94.310762 127.508) (end 94.310762 84.328) (width 0.4) (layer F.Cu) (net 3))
 (segment (start 93.472 79.823301) (end 92.129958 78.481259) (width 0.4) (layer F.Cu) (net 3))
 (segment (start 95.758 136.01192) (end 95.758 134.53872) (width 0.4) (layer F.Cu) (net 3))
 (segment (start 94.310762 133.091482) (end 94.310762 127.508) (width 0.4) (layer F.Cu) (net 3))
 (segment (start 95.758 134.53872) (end 94.310762 133.091482) (width 0.4) (layer F.Cu) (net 3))
 (segment (start 95.758 146.304) (end 93.726 148.336) (width 0.4) (layer F.Cu) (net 3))
 (segment (start 95.758 136.01192) (end 95.758 146.304) (width 0.4) (layer F.Cu) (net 3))
 (segment (start 93.726 148.336) (end 93.472 148.336) (width 0.4) (layer F.Cu) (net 3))
 (segment (start 93.726 148.336) (end 93.2688 148.336) (width 0.25) (layer F.Cu) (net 3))
 (segment (start 94.996 82.804) (end 94.996 82.296) (width 0.4) (layer F.Cu) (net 4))
 (segment (start 94.488 81.788) (end 94.488 79.248) (width 0.4) (layer F.Cu) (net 4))
 (segment (start 94.996 82.296) (end 94.488 81.788) (width 0.4) (layer F.Cu) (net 4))
 (segment (start 94.488 79.248) (end 93.472 78.232) (width 0.4) (layer F.Cu) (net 4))
 (segment (start 93.472 78.232) (end 93.472 74.676) (width 0.4) (layer F.Cu) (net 4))
 (segment (start 93.472 74.676) (end 92.197259 73.401259) (width 0.4) (layer F.Cu) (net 4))
 (segment (start 92.197259 73.401259) (end 92.129958 73.401259) (width 0.4) (layer F.Cu) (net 4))
 (segment (start 92.129958 73.401259) (end 92.197259 73.401259) (width 0.4) (layer F.Cu) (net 4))
 (segment (start 92.197259 73.401259) (end 93.472 74.676) (width 0.4) (layer F.Cu) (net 4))
 (segment (start 94.996 82.804) (end 94.996 123.952) (width 0.4) (layer F.Cu) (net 4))
 (segment (start 94.996 123.952) (end 99.568 128.524) (width 0.4) (layer F.Cu) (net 4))
 (segment (start 99.568 128.524) (end 99.568 131.42976) (width 0.4) (layer F.Cu) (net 4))
 (segment (start 99.568 131.42976) (end 96.4565 134.54126) (width 0.4) (layer F.Cu) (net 4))
 (segment (start 96.4565 148.1455) (end 93.726 150.876) (width 0.4) (layer F.Cu) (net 4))
 (segment (start 96.4565 134.54126) (end 96.4565 148.1455) (width 0.4) (layer F.Cu) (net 4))
 (segment (start 93.726 150.876) (end 93.345 150.876) (width 0.4) (layer F.Cu) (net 4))
 (segment (start 93.726 150.876) (end 93.6625 150.876) (width 0.25) (layer F.Cu) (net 4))
 (segment (start 96.012 81.788) (end 96.012 81.28) (width 0.4) (layer F.Cu) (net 5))
 (segment (start 95.504 80.772) (end 95.504 78.74) (width 0.4) (layer F.Cu) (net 5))
 (segment (start 96.012 81.28) (end 95.504 80.772) (width 0.4) (layer F.Cu) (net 5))
 (segment (start 94.488 77.724) (end 94.488 70.612) (width 0.4) (layer F.Cu) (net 5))
 (segment (start 95.504 78.74) (end 94.488 77.724) (width 0.4) (layer F.Cu) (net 5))
 (segment (start 92.231558 68.092659) (end 92.231558 68.355558) (width 0.4) (layer F.Cu) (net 5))
 (segment (start 92.231558 68.355558) (end 94.488 70.612) (width 0.4) (layer F.Cu) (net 5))
 (segment (start 96.012 81.788) (end 96.012 123.444) (width 0.4) (layer F.Cu) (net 5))
 (segment (start 96.012 123.444) (end 100.584 128.016) (width 0.4) (layer F.Cu) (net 5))
 (segment (start 100.584 128.016) (end 100.584 131.572) (width 0.4) (layer F.Cu) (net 5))
 (segment (start 100.584 131.572) (end 97.536 134.62) (width 0.4) (layer F.Cu) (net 5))
 (segment (start 97.536 134.62) (end 97.536 149.606) (width 0.4) (layer F.Cu) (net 5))
 (segment (start 97.536 149.606) (end 93.726 153.416) (width 0.4) (layer F.Cu) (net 5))
 (segment (start 93.726 153.416) (end 93.55836 153.416) (width 0.25) (layer F.Cu) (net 5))
 (segment (start 93.726 155.956) (end 93.599 155.956) (width 0.4) (layer F.Cu) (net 6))
 (segment (start 93.726 155.956) (end 93.58376 155.956) (width 0.25) (layer F.Cu) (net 6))
 (segment (start 92.202 167.132) (end 93.726 168.656) (width 0.4) (layer F.Cu) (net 11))
 (segment (start 92.202 88.392) (end 92.202 167.132) (width 0.4) (layer F.Cu) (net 11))
 (segment (start 90.932 87.122) (end 92.202 88.392) (width 0.4) (layer F.Cu) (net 11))
 (segment (start 90.932 65.41008) (end 90.932 59.211897) (width 0.4) (layer F.Cu) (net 11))
 (segment (start 90.932 65.41008) (end 90.932 87.122) (width 0.4) (layer F.Cu) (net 11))
 (segment (start 90.932 59.211897) (end 92.221398 57.922499) (width 0.4) (layer F.Cu) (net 11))
 (segment (start 92.329 53.721) (end 92.2655 53.721) (width 0.4) (layer F.Cu) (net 12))
 (segment (start 90.297 60.96508) (end 90.297 54.929457) (width 0.4) (layer F.Cu) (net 12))
 (segment (start 90.297 54.929457) (end 92.297598 52.928859) (width 0.4) (layer F.Cu) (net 12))
 (segment (start 90.297 60.96508) (end 90.297 87.503) (width 0.4) (layer F.Cu) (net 12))
 (segment (start 90.297 87.503) (end 91.567 88.773) (width 0.4) (layer F.Cu) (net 12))
 (segment (start 91.567 88.773) (end 91.567 169.037) (width 0.4) (layer F.Cu) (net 12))
 (segment (start 91.567 169.037) (end 93.726 171.196) (width 0.4) (layer F.Cu) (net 12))
 (segment (start 92.180758 48.052059) (end 92.094981 48.052059) (width 0.4) (layer F.Cu) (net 13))
 (segment (start 92.094981 48.052059) (end 89.63152 50.51552) (width 0.4) (layer F.Cu) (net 13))
 (segment (start 89.63152 50.51552) (end 89.63152 87.706762) (width 0.4) (layer F.Cu) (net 13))
 (segment (start 89.63152 87.706762) (end 90.89136 88.966602) (width 0.4) (layer F.Cu) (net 13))
 (segment (start 90.89136 88.966602) (end 90.89136 170.90136) (width 0.4) (layer F.Cu) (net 13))
 (segment (start 90.89136 170.90136) (end 93.726 173.736) (width 0.4) (layer F.Cu) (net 13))
 (segment (start 97.028 77.724) (end 100.076 77.724) (width 0.4) (layer F.Cu) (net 14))
 (segment (start 100.076 77.724) (end 100.33 77.47) (width 0.4) (layer F.Cu) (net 14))
 (segment (start 100.076 77.724) (end 100.33 77.47) (width 0.4) (layer F.Cu) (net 14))
 (segment (start 97.028 72.644) (end 100.076 72.644) (width 0.4) (layer F.Cu) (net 15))
 (segment (start 100.076 72.644) (end 100.33 72.39) (width 0.4) (layer F.Cu) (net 15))
 (segment (start 97.028 67.564) (end 100.076 67.564) (width 0.4) (layer F.Cu) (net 16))
 (segment (start 100.076 67.564) (end 100.33 67.31) (width 0.4) (layer F.Cu) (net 16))
 (segment (start 97.1296 62.2554) (end 100.3046 62.2554) (width 0.4) (layer F.Cu) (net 17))
 (segment (start 100.3046 62.2554) (end 100.33 62.23) (width 0.4) (layer F.Cu) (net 17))
 (segment (start 97.19564 57.26684) (end 100.4824 57.26684) (width 0.4) (layer F.Cu) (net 18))
 (segment (start 98.4504 52.08016) (end 100.47732 52.08016) (width 0.4) (layer F.Cu) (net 19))
 (segment (start 98.44532 52.08524) (end 98.4504 52.08016) (width 0.4) (layer F.Cu) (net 19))
 (segment (start 97.11944 52.08524) (end 98.44532 52.08524) (width 0.4) (layer F.Cu) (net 19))
 (segment (start 100.41128 47.0916) (end 100.44684 47.05604) (width 0.6) (layer F.Cu) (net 20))
 (segment (start 97.19564 47.0916) (end 100.41128 47.0916) (width 0.4) (layer F.Cu) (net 20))
 (segment (start 97.0788 42.2148) (end 100.4062 42.2148) (width 0.4) (layer F.Cu) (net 21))
 (segment (start 100.4062 42.2148) (end 100.44684 42.25544) (width 0.6) (layer F.Cu) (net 21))
 (segment (start 94.4753 142.5067) (end 93.726 143.256) (width 0.25) (layer F.Cu) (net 1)))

